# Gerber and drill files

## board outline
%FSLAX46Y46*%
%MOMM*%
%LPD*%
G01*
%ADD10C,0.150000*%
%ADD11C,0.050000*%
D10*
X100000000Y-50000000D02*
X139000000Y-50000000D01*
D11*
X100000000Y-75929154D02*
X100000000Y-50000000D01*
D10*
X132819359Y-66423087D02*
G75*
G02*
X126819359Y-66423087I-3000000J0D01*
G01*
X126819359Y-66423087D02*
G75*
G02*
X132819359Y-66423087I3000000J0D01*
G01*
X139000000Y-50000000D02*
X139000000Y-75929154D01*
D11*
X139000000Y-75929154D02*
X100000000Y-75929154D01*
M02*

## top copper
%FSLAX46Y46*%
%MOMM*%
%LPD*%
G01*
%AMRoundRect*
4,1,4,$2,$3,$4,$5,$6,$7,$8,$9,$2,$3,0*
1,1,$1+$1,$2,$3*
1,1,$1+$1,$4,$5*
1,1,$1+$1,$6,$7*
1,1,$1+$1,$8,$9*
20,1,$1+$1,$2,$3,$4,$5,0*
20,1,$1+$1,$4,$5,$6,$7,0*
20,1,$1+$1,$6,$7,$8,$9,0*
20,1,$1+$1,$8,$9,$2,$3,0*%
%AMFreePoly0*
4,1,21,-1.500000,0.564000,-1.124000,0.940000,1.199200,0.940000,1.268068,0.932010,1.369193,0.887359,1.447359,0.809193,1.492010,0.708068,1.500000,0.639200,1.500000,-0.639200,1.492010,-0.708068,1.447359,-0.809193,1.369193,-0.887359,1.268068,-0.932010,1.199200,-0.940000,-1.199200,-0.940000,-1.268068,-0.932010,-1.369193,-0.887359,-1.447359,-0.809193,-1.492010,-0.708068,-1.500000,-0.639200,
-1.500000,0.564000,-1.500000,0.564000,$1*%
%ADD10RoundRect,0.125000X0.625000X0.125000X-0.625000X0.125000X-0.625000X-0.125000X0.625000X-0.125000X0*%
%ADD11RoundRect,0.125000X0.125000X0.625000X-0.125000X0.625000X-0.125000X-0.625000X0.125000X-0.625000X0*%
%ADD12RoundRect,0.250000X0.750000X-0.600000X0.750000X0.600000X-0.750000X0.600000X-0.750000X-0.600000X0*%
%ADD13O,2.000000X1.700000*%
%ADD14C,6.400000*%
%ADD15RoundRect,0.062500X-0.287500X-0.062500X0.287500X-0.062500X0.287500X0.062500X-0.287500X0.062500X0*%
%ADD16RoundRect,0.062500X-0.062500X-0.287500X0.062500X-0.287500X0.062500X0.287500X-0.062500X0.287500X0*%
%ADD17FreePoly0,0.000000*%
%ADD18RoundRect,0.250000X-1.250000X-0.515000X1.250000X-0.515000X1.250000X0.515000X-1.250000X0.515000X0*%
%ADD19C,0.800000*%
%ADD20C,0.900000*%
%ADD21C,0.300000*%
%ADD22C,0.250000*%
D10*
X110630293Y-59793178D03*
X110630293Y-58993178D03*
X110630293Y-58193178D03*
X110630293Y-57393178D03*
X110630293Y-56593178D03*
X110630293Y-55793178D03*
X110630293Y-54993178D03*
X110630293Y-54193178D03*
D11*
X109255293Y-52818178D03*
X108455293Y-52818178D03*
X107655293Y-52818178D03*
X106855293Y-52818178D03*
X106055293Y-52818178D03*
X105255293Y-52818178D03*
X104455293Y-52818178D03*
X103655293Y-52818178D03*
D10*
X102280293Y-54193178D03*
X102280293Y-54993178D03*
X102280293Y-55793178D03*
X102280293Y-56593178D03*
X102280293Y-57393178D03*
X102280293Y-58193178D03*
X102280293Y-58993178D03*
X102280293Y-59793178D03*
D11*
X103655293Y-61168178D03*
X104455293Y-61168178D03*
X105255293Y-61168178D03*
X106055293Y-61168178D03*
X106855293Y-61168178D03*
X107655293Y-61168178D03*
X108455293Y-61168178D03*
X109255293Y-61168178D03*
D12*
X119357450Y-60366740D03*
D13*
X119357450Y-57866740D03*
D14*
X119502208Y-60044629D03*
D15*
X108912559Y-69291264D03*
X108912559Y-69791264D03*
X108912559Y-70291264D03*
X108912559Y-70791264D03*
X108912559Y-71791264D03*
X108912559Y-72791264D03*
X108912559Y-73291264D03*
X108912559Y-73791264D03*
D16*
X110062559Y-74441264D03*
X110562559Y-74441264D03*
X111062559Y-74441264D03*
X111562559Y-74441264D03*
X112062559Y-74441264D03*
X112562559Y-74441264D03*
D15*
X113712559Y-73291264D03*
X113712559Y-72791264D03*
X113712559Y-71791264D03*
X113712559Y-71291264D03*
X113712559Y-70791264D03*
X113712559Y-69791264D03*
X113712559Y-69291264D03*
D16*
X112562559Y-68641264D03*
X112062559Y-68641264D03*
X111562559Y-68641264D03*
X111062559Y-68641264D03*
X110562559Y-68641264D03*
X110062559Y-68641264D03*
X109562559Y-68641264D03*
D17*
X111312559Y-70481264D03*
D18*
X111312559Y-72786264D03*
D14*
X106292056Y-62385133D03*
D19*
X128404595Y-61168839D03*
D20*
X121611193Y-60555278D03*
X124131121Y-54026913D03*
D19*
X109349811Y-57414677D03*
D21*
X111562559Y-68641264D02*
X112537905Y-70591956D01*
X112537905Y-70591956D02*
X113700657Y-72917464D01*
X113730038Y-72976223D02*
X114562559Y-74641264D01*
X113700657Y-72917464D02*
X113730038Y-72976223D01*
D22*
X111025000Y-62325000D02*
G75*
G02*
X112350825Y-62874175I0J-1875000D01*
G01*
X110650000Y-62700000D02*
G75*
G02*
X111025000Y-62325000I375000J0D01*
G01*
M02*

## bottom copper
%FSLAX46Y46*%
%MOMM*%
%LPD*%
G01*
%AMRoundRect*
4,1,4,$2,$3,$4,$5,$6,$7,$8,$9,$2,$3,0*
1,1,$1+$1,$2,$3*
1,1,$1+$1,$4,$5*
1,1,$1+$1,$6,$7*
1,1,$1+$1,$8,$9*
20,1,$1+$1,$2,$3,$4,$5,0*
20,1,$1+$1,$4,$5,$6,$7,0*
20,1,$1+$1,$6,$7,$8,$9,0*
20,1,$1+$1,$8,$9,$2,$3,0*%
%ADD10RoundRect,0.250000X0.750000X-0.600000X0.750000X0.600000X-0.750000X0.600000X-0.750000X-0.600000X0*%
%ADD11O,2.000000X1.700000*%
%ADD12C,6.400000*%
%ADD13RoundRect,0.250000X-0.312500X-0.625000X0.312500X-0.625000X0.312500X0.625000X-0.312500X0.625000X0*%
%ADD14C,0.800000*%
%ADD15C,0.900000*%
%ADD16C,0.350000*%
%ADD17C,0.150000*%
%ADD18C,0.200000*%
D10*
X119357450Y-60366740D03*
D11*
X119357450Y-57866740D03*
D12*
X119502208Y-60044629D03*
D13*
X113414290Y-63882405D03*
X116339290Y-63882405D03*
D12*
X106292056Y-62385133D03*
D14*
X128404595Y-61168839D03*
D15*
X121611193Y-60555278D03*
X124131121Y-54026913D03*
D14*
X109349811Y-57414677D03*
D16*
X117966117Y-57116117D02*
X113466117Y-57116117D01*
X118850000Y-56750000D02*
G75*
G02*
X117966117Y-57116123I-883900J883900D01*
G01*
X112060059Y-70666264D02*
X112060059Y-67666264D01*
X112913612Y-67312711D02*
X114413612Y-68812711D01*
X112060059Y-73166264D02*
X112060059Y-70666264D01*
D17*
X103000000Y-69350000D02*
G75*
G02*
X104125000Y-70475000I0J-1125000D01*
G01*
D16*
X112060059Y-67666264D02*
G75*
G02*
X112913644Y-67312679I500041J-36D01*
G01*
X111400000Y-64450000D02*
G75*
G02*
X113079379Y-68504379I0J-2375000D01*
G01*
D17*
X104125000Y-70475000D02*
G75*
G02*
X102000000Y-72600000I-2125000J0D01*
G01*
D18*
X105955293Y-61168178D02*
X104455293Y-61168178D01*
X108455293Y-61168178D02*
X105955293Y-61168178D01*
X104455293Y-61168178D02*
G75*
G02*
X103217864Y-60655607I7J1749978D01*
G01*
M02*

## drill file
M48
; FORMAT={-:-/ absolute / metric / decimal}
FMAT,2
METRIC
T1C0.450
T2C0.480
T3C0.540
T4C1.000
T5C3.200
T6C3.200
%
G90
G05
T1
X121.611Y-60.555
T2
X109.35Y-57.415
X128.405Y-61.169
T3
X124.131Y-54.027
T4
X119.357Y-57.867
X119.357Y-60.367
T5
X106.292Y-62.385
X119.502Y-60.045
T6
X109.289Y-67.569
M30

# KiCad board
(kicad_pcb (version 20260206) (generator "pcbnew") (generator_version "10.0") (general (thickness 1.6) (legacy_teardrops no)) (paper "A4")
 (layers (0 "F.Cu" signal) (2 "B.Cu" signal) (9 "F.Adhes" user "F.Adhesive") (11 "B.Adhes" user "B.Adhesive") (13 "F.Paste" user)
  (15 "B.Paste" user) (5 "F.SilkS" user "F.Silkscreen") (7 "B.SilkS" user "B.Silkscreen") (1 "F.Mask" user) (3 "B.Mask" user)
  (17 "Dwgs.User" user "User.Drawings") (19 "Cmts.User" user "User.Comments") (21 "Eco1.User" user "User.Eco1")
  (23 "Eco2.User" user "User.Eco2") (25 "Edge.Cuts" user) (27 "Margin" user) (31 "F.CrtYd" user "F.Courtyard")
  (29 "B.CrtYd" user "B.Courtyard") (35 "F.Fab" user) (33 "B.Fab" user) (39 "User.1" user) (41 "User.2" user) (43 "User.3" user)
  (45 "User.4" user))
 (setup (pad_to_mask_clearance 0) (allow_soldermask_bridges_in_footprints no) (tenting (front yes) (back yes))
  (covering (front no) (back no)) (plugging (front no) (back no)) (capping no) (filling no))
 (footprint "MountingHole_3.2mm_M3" (layer "F.Cu") (at 109.289246 67.568769)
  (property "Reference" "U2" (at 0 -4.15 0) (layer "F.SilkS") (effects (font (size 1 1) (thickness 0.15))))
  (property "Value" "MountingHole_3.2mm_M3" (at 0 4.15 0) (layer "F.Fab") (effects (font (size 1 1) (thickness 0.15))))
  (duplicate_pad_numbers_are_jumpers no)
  (pad "" np_thru_hole circle (at 0 0) (size 3.2 3.2) (drill 3.2) (layers "*.Cu" "*.Mask")))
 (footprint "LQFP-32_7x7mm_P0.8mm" (layer "F.Cu") (at 106.455293 56.993178 180)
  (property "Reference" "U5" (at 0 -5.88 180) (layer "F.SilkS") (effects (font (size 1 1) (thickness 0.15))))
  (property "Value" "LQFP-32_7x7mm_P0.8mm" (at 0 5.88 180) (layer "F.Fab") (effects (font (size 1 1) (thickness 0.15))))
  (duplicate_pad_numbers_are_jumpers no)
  (pad "1" smd roundrect (at -4.175 -2.8 180) (size 1.5 0.5) (layers "F.Cu" "F.Mask" "F.Paste") (roundrect_rratio 0.25) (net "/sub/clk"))
  (pad "2" smd roundrect (at -4.175 -2 180) (size 1.5 0.5) (layers "F.Cu" "F.Mask" "F.Paste") (roundrect_rratio 0.25) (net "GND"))
  (pad "3" smd roundrect (at -4.175 -1.2 180) (size 1.5 0.5) (layers "F.Cu" "F.Mask" "F.Paste") (roundrect_rratio 0.25) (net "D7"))
  (pad "4" smd roundrect (at -4.175 -0.4 180) (size 1.5 0.5) (layers "F.Cu" "F.Mask" "F.Paste") (roundrect_rratio 0.25) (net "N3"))
  (pad "5" smd roundrect (at -4.175 0.4 180) (size 1.5 0.5) (layers "F.Cu" "F.Mask" "F.Paste") (roundrect_rratio 0.25))
  (pad "6" smd roundrect (at -4.175 1.2 180) (size 1.5 0.5) (layers "F.Cu" "F.Mask" "F.Paste") (roundrect_rratio 0.25) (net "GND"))
  (pad "7" smd roundrect (at -4.175 2 180) (size 1.5 0.5) (layers "F.Cu" "F.Mask" "F.Paste") (roundrect_rratio 0.25))
  (pad "8" smd roundrect (at -4.175 2.8 180) (size 1.5 0.5) (layers "F.Cu" "F.Mask" "F.Paste") (roundrect_rratio 0.25) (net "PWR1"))
  (pad "9" smd roundrect (at -2.8 4.175 180) (size 0.5 1.5) (layers "F.Cu" "F.Mask" "F.Paste") (roundrect_rratio 0.25) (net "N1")
   (clearance 0.35))
  (pad "10" smd roundrect (at -2 4.175 180) (size 0.5 1.5) (layers "F.Cu" "F.Mask" "F.Paste") (roundrect_rratio 0.25) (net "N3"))
  (pad "11" smd roundrect (at -1.2 4.175 180) (size 0.5 1.5) (layers "F.Cu" "F.Mask" "F.Paste") (roundrect_rratio 0.25) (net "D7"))
  (pad "12" smd roundrect (at -0.4 4.175 180) (size 0.5 1.5) (layers "F.Cu" "F.Mask" "F.Paste") (roundrect_rratio 0.25) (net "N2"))
  (pad "13" smd roundrect (at 0.4 4.175 180) (size 0.5 1.5) (layers "F.Cu" "F.Mask" "F.Paste") (roundrect_rratio 0.25) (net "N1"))
  (pad "14" smd roundrect (at 1.2 4.175 180) (size 0.5 1.5) (layers "F.Cu" "F.Mask" "F.Paste") (roundrect_rratio 0.25) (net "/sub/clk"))
  (pad "15" smd roundrect (at 2 4.175 180) (size 0.5 1.5) (layers "F.Cu" "F.Mask" "F.Paste") (roundrect_rratio 0.25))
  (pad "16" smd roundrect (at 2.8 4.175 180) (size 0.5 1.5) (layers "F.Cu" "F.Mask" "F.Paste") (roundrect_rratio 0.25))
  (pad "17" smd roundrect (at 4.175 2.8 180) (size 1.5 0.5) (layers "F.Cu" "F.Mask" "F.Paste") (roundrect_rratio 0.25) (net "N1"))
  (pad "18" smd roundrect (at 4.175 2 180) (size 1.5 0.5) (layers "F.Cu" "F.Mask" "F.Paste") (roundrect_rratio 0.25) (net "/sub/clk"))
  (pad "19" smd roundrect (at 4.175 1.2 180) (size 1.5 0.5) (layers "F.Cu" "F.Mask" "F.Paste") (roundrect_rratio 0.25) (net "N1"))
  (pad "20" smd roundrect (at 4.175 0.4 180) (size 1.5 0.5) (layers "F.Cu" "F.Mask" "F.Paste") (roundrect_rratio 0.25) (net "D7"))
  (pad "21" smd roundrect (at 4.175 -0.4 180) (size 1.5 0.5) (layers "F.Cu" "F.Mask" "F.Paste") (roundrect_rratio 0.25) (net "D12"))
  (pad "22" smd roundrect (at 4.175 -1.2 180) (size 1.5 0.5) (layers "F.Cu" "F.Mask" "F.Paste") (roundrect_rratio 0.25))
  (pad "23" smd roundrect (at 4.175 -2 180) (size 1.5 0.5) (layers "F.Cu" "F.Mask" "F.Paste") (roundrect_rratio 0.25))
  (pad "24" smd roundrect (at 4.175 -2.8 180) (size 1.5 0.5) (layers "F.Cu" "F.Mask" "F.Paste") (roundrect_rratio 0.25))
  (pad "25" smd roundrect (at 2.8 -4.175 180) (size 0.5 1.5) (layers "F.Cu" "F.Mask" "F.Paste") (roundrect_rratio 0.25) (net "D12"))
  (pad "26" smd roundrect (at 2 -4.175 180) (size 0.5 1.5) (layers "F.Cu" "F.Mask" "F.Paste") (roundrect_rratio 0.25) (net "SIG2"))
  (pad "27" smd roundrect (at 1.2 -4.175 180) (size 0.5 1.5) (layers "F.Cu" "F.Mask" "F.Paste") (roundrect_rratio 0.25) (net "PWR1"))
  (pad "28" smd roundrect (at 0.4 -4.175 180) (size 0.5 1.5) (layers "F.Cu" "F.Mask" "F.Paste") (roundrect_rratio 0.25) (clearance 0.35))
  (pad "29" smd roundrect (at -0.4 -4.175 180) (size 0.5 1.5) (layers "F.Cu" "F.Mask" "F.Paste") (roundrect_rratio 0.25) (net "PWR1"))
  (pad "30" smd roundrect (at -1.2 -4.175 180) (size 0.5 1.5) (layers "F.Cu" "F.Mask" "F.Paste") (roundrect_rratio 0.25) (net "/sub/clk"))
  (pad "31" smd roundrect (at -2 -4.175 180) (size 0.5 1.5) (layers "F.Cu" "F.Mask" "F.Paste") (roundrect_rratio 0.25) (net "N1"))
  (pad "32" smd roundrect (at -2.8 -4.175 180) (size 0.5 1.5) (layers "F.Cu" "F.Mask" "F.Paste") (roundrect_rratio 0.25) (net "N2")))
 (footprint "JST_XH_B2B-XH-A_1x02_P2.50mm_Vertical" (layer "F.Cu") (at 119.35745 60.36674 90)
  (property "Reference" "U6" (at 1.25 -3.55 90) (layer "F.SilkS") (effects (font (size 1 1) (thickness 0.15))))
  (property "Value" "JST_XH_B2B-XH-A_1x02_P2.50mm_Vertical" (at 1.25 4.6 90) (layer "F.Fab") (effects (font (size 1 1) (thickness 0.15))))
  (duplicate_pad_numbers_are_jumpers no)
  (pad "1" thru_hole roundrect (at 0 0 90) (size 1.7 2) (drill 1) (layers "*.Cu" "*.Mask") (remove_unused_layers no)
   (roundrect_rratio 0.147059) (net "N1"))
  (pad "2" thru_hole oval (at 2.5 0 90) (size 1.7 2) (drill 1) (layers "*.Cu" "*.Mask") (remove_unused_layers no)))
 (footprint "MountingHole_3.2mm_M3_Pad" (layer "F.Cu") (at 119.502208 60.044629)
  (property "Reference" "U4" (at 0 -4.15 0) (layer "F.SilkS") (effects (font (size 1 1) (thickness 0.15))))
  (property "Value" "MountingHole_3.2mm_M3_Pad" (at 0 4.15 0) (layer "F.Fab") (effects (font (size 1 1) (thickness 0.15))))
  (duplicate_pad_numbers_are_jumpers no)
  (pad "1" thru_hole circle (at 0 0) (size 6.4 6.4) (drill 3.2) (layers "*.Cu" "*.Mask") (remove_unused_layers no) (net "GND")
   (zone_connect 2)))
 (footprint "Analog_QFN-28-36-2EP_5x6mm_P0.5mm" (layer "F.Cu") (at 111.312559 71.541264)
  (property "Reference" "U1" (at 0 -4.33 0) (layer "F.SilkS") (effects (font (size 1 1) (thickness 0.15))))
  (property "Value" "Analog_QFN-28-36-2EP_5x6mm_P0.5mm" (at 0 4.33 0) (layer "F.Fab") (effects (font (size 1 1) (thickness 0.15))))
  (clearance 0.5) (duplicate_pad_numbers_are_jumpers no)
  (pad "" smd roundrect (at -0.75 -1.53) (size 1.21 0.76) (layers "F.Paste") (roundrect_rratio 0.25) (chamfer_ratio 0.4) (chamfer top_left)
   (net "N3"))
  (pad "" smd roundrect (at -0.75 -0.59) (size 1.21 0.76) (layers "F.Paste") (roundrect_rratio 0.25) (clearance 0.1))
  (pad "" smd roundrect (at -0.7475 0.875) (size 1.205 0.55) (layers "F.Paste") (roundrect_rratio 0.25) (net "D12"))
  (pad "" smd roundrect (at -0.7475 1.625) (size 1.205 0.55) (layers "F.Paste") (roundrect_rratio 0.25) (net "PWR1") (clearance 0.35))
  (pad "" smd roundrect (at 0.7475 0.875) (size 1.205 0.55) (layers "F.Paste") (roundrect_rratio 0.25) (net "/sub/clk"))
  (pad "" smd roundrect (at 0.7475 1.625) (size 1.205 0.55) (layers "F.Paste") (roundrect_rratio 0.25) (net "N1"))
  (pad "" smd roundrect (at 0.75 -1.53) (size 1.21 0.76) (layers "F.Paste") (roundrect_rratio 0.25) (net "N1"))
  (pad "" smd roundrect (at 0.75 -0.59) (size 1.21 0.76) (layers "F.Paste") (roundrect_rratio 0.25) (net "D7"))
  (pad "1" smd roundrect (at -2.4 -2.25) (size 0.7 0.25) (layers "F.Cu" "F.Mask" "F.Paste") (roundrect_rratio 0.25) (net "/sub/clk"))
  (pad "2" smd roundrect (at -2.4 -1.75) (size 0.7 0.25) (layers "F.Cu" "F.Mask" "F.Paste") (roundrect_rratio 0.25) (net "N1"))
  (pad "3" smd roundrect (at -2.4 -1.25) (size 0.7 0.25) (layers "F.Cu" "F.Mask" "F.Paste") (roundrect_rratio 0.25))
  (pad "4" smd roundrect (at -2.4 -0.75) (size 0.7 0.25) (layers "F.Cu" "F.Mask" "F.Paste") (roundrect_rratio 0.25))
  (pad "6" smd roundrect (at -2.4 0.25) (size 0.7 0.25) (layers "F.Cu" "F.Mask" "F.Paste") (roundrect_rratio 0.25) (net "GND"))
  (pad "8" smd roundrect (at -2.4 1.25) (size 0.7 0.25) (layers "F.Cu" "F.Mask" "F.Paste") (roundrect_rratio 0.25))
  (pad "9" smd roundrect (at -2.4 1.75) (size 0.7 0.25) (layers "F.Cu" "F.Mask" "F.Paste") (roundrect_rratio 0.25) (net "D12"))
  (pad "10" smd roundrect (at -2.4 2.25) (size 0.7 0.25) (layers "F.Cu" "F.Mask" "F.Paste") (roundrect_rratio 0.25) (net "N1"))
  (pad "12" smd roundrect (at -1.25 2.9) (size 0.25 0.7) (layers "F.Cu" "F.Mask" "F.Paste") (roundrect_rratio 0.25))
  (pad "13" smd roundrect (at -0.75 2.9) (size 0.25 0.7) (layers "F.Cu" "F.Mask" "F.Paste") (roundrect_rratio 0.25) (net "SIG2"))
  (pad "14" smd roundrect (at -0.25 2.9) (size 0.25 0.7) (layers "F.Cu" "F.Mask" "F.Paste") (roundrect_rratio 0.25) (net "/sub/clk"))
  (pad "15" smd roundrect (at 0.25 2.9) (size 0.25 0.7) (layers "F.Cu" "F.Mask" "F.Paste") (roundrect_rratio 0.25))
  (pad "16" smd roundrect (at 0.75 2.9) (size 0.25 0.7) (layers "F.Cu" "F.Mask" "F.Paste") (roundrect_rratio 0.25) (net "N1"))
  (pad "17" smd roundrect (at 1.25 2.9) (size 0.25 0.7) (layers "F.Cu" "F.Mask" "F.Paste") (roundrect_rratio 0.25) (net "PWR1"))
  (pad "20" smd roundrect (at 2.4 1.75) (size 0.7 0.25) (layers "F.Cu" "F.Mask" "F.Paste") (roundrect_rratio 0.25) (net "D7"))
  (pad "21" smd roundrect (at 2.4 1.25) (size 0.7 0.25) (layers "F.Cu" "F.Mask" "F.Paste") (roundrect_rratio 0.25) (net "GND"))
  (pad "23" smd roundrect (at 2.4 0.25) (size 0.7 0.25) (layers "F.Cu" "F.Mask" "F.Paste") (roundrect_rratio 0.25))
  (pad "24" smd roundrect (at 2.4 -0.25) (size 0.7 0.25) (layers "F.Cu" "F.Mask" "F.Paste") (roundrect_rratio 0.25) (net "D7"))
  (pad "25" smd roundrect (at 2.4 -0.75) (size 0.7 0.25) (layers "F.Cu" "F.Mask" "F.Paste") (roundrect_rratio 0.25) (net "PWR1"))
  (pad "27" smd roundrect (at 2.4 -1.75) (size 0.7 0.25) (layers "F.Cu" "F.Mask" "F.Paste") (roundrect_rratio 0.25) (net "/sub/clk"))
  (pad "28" smd roundrect (at 2.4 -2.25) (size 0.7 0.25) (layers "F.Cu" "F.Mask" "F.Paste") (roundrect_rratio 0.25) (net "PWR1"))
  (pad "30" smd roundrect (at 1.25 -2.9) (size 0.25 0.7) (layers "F.Cu" "F.Mask" "F.Paste") (roundrect_rratio 0.25))
  (pad "31" smd roundrect (at 0.75 -2.9) (size 0.25 0.7) (layers "F.Cu" "F.Mask" "F.Paste") (roundrect_rratio 0.25))
  (pad "32" smd roundrect (at 0.25 -2.9) (size 0.25 0.7) (layers "F.Cu" "F.Mask" "F.Paste") (roundrect_rratio 0.25))
  (pad "33" smd roundrect (at -0.25 -2.9) (size 0.25 0.7) (layers "F.Cu" "F.Mask" "F.Paste") (roundrect_rratio 0.25) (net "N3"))
  (pad "34" smd roundrect (at -0.75 -2.9) (size 0.25 0.7) (layers "F.Cu" "F.Mask" "F.Paste") (roundrect_rratio 0.25))
  (pad "35" smd roundrect (at -1.25 -2.9) (size 0.25 0.7) (layers "F.Cu" "F.Mask" "F.Paste") (roundrect_rratio 0.25))
  (pad "36" smd roundrect (at -1.75 -2.9) (size 0.25 0.7) (layers "F.Cu" "F.Mask" "F.Paste") (roundrect_rratio 0.25) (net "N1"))
  (pad "37" smd roundrect (at 0 -1.06) (size 3 1.88) (layers "F.Cu" "F.Mask") (roundrect_rratio 0.16) (chamfer_ratio 0.2) (chamfer top_left)
   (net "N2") (zone_connect 2))
  (pad "38" smd roundrect (at 0 1.245) (size 3 1.53) (layers "F.Cu" "F.Mask") (roundrect_rratio 0.1633986928) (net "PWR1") (zone_connect 2)))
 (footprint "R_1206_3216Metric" (layer "B.Cu") (at 114.87679 63.882405)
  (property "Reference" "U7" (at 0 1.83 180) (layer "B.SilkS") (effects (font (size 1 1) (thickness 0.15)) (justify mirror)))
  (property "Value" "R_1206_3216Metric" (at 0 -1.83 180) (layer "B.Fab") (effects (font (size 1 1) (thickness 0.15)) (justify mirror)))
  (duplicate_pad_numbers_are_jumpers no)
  (pad "1" smd roundrect (at -1.4625 0) (size 1.125 1.75) (layers "B.Cu" "B.Mask" "B.Paste") (roundrect_rratio 0.222222) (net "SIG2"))
  (pad "2" smd roundrect (at 1.4625 0) (size 1.125 1.75) (layers "B.Cu" "B.Mask" "B.Paste") (roundrect_rratio 0.222222) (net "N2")))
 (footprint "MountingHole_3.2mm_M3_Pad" (layer "B.Cu") (at 106.292056 62.385133 90)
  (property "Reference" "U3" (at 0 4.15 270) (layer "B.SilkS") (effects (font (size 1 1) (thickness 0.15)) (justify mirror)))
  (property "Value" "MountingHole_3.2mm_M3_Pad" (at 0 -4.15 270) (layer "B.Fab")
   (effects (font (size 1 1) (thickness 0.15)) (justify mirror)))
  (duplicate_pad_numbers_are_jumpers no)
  (pad "1" thru_hole circle (at 0 0 90) (size 6.4 6.4) (drill 3.2) (layers "*.Cu" "*.Mask") (remove_unused_layers no) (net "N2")
   (clearance 0.1) (zone_connect 2)))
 (gr_line (start 100 50) (end 139 50) (stroke (width 0.15) (type default)) (layer "Edge.Cuts"))
 (gr_line (start 100 75.929154) (end 100 50) (stroke (width 0.05) (type default)) (layer "Edge.Cuts"))
 (gr_circle (center 129.819359 66.423087) (end 132.819359 66.423087) (stroke (width 0.15) (type default)) (fill no) (layer "Edge.Cuts"))
 (gr_line (start 139 50) (end 139 75.929154) (stroke (width 0.15) (type default)) (layer "Edge.Cuts"))
 (gr_line (start 139 75.929154) (end 100 75.929154) (stroke (width 0.05) (type default)) (layer "Edge.Cuts"))
 (segment (start 111.562559 68.641264) (end 112.537905 70.591956) (width 0.3) (layer "F.Cu") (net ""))
 (segment (start 112.537905 70.591956) (end 113.700657 72.917464) (width 0.3) (layer "F.Cu") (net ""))
 (segment (start 113.730038 72.976223) (end 114.562559 74.641264) (width 0.3) (layer "F.Cu") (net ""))
 (segment (start 113.700657 72.917464) (end 113.730038 72.976223) (width 0.3) (layer "F.Cu") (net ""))
 (arc (start 111.025 62.325) (mid 111.742531 62.467726) (end 112.350825 62.874175) (width 0.25) (locked yes) (layer "F.Cu") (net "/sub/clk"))
 (arc (start 110.65 62.7) (mid 110.759835 62.434835) (end 111.025 62.325) (width 0.25) (layer "F.Cu") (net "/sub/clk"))
 (via (at 128.404595 61.168839) (size 0.8) (drill 0.48) (layers "F.Cu" "B.Cu") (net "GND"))
 (via (at 121.611193 60.555278) (size 0.9) (drill 0.45) (layers "F.Cu" "B.Cu") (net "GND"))
 (segment (start 117.966117 57.116117) (end 113.466117 57.116117) (width 0.35) (layer "B.Cu") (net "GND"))
 (arc (start 118.85 56.75) (mid 118.444471 57.020966) (end 117.966117 57.116117) (width 0.35) (layer "B.Cu") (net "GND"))
 (via (at 124.131121 54.026913) (size 0.9) (drill 0.54) (layers "F.Cu" "B.Cu") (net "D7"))
 (via (at 109.349811 57.414677) (size 0.8) (drill 0.48) (layers "F.Cu" "B.Cu") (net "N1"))
 (segment (start 112.060059 70.666264) (end 112.060059 67.666264) (width 0.35) (layer "B.Cu") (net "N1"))
 (segment (start 112.913612 67.312711) (end 114.413612 68.812711) (width 0.35) (layer "B.Cu") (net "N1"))
 (segment (start 112.060059 73.166264) (end 112.060059 70.666264) (width 0.35) (layer "B.Cu") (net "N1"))
 (arc (start 103 69.35) (mid 103.795495 69.679505) (end 104.125 70.475) (width 0.15) (layer "B.Cu") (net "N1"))
 (arc (start 112.060059 67.666264) (mid 112.368717 67.204324) (end 112.913612 67.312711) (width 0.35) (layer "B.Cu") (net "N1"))
 (arc (start 111.4 64.45) (mid 113.594214 65.916127) (end 113.079379 68.504379) (width 0.35) (layer "B.Cu") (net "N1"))
 (arc (start 104.125 70.475) (mid 103.502602 71.977602) (end 102 72.6) (width 0.15) (locked yes) (layer "B.Cu") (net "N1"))
 (segment (start 105.955293 61.168178) (end 104.455293 61.168178) (width 0.2) (layer "B.Cu") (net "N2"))
 (segment (start 108.455293 61.168178) (end 105.955293 61.168178) (width 0.2) (layer "B.Cu") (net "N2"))
 (arc (start 104.455293 61.168178) (mid 103.785597 61.034967) (end 103.217856 60.655615) (width 0.2) (layer "B.Cu") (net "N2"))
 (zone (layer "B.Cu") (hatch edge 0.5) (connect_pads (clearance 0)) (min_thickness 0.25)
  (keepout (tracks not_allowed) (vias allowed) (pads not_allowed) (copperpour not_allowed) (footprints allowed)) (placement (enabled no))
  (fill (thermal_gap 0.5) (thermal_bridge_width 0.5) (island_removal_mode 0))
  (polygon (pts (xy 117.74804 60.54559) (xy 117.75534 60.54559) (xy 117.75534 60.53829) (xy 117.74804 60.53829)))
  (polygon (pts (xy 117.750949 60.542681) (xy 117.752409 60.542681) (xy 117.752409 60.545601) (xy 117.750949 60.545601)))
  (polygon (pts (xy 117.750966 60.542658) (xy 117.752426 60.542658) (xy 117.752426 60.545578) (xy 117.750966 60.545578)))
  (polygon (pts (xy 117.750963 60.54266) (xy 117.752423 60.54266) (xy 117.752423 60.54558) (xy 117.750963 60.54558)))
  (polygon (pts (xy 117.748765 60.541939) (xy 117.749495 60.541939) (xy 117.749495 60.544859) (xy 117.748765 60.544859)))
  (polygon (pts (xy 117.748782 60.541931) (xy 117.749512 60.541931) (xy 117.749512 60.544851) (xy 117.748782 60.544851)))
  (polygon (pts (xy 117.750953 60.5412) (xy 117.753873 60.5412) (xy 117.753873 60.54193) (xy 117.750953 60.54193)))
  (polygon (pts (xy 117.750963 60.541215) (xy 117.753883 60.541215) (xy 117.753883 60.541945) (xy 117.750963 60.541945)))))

